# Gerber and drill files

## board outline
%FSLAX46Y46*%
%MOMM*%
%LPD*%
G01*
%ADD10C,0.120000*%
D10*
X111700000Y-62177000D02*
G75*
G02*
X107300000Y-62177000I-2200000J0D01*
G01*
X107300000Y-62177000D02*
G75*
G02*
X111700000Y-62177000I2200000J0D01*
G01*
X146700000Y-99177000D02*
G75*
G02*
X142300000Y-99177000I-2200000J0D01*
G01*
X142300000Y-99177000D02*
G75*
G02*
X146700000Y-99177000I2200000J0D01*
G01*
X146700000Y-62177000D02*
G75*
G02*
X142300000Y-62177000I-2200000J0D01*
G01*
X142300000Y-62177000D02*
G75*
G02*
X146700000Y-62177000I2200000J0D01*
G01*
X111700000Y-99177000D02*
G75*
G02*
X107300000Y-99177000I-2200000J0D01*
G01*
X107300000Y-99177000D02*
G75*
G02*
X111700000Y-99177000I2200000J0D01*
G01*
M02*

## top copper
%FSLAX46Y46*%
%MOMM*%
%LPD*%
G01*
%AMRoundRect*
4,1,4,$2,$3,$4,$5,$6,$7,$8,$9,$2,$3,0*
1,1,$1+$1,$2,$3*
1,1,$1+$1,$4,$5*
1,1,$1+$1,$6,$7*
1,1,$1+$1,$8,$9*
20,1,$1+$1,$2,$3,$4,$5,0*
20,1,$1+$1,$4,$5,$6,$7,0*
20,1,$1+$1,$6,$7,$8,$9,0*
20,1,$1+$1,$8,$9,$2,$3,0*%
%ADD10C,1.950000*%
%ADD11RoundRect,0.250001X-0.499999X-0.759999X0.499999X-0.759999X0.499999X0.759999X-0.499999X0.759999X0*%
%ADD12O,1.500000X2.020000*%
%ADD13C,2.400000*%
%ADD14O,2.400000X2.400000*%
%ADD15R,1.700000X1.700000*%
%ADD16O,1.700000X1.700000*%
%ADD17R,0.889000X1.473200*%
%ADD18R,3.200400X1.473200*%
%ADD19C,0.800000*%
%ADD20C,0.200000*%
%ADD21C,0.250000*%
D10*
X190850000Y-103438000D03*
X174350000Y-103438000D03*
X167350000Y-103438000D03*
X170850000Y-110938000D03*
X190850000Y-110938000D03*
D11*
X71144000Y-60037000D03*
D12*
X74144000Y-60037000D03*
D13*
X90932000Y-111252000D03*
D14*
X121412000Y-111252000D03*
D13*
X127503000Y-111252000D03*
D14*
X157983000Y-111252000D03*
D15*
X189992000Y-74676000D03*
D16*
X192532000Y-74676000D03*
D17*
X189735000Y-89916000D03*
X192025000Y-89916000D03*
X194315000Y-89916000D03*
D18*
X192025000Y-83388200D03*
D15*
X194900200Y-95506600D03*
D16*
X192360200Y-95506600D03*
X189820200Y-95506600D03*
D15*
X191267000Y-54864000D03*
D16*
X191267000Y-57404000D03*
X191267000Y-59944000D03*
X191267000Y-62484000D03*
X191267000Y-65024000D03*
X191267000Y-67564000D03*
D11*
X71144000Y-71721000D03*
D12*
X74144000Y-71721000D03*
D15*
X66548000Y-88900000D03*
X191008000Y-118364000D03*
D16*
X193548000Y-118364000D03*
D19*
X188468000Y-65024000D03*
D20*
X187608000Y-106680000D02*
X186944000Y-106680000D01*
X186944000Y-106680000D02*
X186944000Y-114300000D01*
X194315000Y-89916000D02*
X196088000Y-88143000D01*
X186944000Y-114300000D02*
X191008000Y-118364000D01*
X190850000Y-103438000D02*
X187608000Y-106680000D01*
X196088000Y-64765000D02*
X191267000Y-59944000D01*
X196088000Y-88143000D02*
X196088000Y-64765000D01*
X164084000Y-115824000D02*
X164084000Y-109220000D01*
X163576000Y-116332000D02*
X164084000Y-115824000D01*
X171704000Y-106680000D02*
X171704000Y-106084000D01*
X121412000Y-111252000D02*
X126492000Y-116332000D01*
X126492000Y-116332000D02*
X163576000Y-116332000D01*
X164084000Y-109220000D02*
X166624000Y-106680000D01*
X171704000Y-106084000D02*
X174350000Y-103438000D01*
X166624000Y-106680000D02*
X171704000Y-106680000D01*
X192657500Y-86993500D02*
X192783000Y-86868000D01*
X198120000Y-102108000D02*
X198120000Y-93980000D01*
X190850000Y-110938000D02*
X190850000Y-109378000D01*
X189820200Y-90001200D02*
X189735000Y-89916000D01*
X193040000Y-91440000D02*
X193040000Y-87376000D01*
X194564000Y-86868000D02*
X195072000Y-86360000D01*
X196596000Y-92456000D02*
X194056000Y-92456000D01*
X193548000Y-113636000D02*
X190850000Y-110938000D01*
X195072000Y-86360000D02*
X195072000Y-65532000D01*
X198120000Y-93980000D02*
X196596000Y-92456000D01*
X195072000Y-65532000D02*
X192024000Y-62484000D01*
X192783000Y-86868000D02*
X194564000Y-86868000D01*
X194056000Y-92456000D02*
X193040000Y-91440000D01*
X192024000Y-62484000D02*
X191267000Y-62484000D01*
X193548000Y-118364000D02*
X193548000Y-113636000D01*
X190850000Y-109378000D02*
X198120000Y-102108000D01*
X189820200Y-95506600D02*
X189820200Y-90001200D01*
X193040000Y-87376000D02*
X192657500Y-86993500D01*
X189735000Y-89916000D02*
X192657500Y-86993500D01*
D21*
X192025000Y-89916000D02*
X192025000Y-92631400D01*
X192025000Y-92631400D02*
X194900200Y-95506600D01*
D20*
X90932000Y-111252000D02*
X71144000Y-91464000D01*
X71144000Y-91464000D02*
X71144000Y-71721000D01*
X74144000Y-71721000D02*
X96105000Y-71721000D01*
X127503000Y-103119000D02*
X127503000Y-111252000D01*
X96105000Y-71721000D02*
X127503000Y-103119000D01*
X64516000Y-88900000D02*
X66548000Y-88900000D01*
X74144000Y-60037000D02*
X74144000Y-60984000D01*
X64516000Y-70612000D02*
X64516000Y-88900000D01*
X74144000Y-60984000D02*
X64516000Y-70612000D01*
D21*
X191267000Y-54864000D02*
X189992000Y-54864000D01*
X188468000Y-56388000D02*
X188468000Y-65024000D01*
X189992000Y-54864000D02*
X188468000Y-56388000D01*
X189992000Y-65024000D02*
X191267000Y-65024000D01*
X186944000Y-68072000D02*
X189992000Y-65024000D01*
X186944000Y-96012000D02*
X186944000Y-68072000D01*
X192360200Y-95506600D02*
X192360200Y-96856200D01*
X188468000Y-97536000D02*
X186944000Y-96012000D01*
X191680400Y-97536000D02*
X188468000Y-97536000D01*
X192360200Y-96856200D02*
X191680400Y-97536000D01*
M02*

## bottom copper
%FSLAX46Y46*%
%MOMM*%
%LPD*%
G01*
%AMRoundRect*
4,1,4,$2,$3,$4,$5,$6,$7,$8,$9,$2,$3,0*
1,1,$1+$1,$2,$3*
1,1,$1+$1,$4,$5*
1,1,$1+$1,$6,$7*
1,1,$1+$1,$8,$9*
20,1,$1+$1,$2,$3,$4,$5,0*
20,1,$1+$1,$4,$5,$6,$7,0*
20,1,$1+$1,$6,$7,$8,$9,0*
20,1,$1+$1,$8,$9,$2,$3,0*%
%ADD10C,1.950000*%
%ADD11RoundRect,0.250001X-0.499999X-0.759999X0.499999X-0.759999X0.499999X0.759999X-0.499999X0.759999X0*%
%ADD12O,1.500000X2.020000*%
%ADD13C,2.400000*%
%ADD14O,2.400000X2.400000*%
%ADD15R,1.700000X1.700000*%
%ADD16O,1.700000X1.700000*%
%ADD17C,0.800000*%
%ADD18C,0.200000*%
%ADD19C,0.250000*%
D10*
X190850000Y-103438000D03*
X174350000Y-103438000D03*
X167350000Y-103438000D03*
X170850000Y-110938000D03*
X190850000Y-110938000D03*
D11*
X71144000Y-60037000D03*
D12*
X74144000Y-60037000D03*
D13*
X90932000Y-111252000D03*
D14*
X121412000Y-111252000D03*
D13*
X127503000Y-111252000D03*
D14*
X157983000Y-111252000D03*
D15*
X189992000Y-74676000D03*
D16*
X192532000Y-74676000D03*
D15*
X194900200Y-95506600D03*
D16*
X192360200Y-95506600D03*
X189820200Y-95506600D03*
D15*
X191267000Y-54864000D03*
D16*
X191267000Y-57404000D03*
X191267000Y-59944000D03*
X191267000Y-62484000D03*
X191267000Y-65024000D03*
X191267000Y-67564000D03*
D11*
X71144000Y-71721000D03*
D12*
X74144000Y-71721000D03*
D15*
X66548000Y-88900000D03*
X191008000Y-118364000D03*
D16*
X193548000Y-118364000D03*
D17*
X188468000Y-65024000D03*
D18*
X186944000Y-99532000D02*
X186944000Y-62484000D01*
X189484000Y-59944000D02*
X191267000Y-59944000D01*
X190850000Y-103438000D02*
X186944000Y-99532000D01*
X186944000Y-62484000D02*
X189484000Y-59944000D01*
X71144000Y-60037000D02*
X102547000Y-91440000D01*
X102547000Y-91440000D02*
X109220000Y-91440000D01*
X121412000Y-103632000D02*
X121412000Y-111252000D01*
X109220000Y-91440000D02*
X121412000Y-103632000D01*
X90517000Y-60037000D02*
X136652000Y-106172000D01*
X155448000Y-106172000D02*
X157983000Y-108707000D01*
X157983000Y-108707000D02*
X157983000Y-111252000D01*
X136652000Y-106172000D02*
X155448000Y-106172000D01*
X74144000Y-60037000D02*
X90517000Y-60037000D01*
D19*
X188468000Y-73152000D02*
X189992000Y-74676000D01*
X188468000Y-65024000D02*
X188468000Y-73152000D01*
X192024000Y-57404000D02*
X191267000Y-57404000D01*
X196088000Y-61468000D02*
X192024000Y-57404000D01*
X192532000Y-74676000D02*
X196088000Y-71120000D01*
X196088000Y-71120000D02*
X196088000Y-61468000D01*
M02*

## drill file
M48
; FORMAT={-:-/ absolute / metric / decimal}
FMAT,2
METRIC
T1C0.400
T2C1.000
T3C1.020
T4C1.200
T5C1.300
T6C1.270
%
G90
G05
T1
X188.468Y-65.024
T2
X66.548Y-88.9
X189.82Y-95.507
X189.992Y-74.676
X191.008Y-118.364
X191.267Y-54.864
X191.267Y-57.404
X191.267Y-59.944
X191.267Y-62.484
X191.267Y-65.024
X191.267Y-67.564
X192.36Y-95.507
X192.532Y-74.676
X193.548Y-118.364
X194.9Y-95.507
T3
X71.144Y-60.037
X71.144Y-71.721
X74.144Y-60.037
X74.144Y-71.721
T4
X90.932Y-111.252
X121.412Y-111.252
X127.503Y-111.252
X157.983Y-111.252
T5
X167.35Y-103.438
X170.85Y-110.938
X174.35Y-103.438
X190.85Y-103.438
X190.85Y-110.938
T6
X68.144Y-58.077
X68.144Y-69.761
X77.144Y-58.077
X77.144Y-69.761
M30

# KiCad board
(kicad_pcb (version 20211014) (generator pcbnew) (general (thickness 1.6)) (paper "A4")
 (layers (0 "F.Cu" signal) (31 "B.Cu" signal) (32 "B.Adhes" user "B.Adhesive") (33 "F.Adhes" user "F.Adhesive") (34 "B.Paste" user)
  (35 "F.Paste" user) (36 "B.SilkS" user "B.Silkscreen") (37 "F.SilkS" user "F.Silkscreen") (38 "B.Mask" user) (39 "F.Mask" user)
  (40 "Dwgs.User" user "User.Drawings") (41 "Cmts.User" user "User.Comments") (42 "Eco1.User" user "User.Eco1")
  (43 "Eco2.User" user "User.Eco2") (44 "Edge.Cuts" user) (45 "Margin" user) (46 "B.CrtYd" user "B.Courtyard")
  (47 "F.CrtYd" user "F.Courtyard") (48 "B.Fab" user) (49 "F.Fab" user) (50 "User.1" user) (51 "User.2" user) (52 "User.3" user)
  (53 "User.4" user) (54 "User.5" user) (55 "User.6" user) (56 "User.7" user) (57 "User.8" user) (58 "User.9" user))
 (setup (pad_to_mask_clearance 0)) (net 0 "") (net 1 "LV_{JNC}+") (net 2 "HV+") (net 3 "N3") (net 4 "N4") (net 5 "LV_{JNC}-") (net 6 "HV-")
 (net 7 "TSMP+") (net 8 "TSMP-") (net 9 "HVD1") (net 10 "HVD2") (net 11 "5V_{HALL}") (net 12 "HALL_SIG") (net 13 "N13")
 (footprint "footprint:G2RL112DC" (layer "F.Cu") (at 190.85 103.438 180)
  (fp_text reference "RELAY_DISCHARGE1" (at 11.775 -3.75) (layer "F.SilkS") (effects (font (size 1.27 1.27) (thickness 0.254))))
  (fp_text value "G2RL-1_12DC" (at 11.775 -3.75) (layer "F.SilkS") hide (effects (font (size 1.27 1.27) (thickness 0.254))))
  (pad "1" thru_hole circle (at 0 0 180) (size 1.95 1.95) (drill 1.3) (layers *.Cu *.Mask) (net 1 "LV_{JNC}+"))
  (pad "2" thru_hole circle (at 16.5 0 180) (size 1.95 1.95) (drill 1.3) (layers *.Cu *.Mask) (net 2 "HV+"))
  (pad "3" thru_hole circle (at 23.5 0 180) (size 1.95 1.95) (drill 1.3) (layers *.Cu *.Mask) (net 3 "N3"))
  (pad "4" thru_hole circle (at 20 -7.5 180) (size 1.95 1.95) (drill 1.3) (layers *.Cu *.Mask) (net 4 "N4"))
  (pad "5" thru_hole circle (at 0 -7.5 180) (size 1.95 1.95) (drill 1.3) (layers *.Cu *.Mask) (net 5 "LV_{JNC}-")))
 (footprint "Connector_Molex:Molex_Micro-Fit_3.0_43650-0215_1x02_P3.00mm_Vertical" (layer "F.Cu") (at 71.144 60.037)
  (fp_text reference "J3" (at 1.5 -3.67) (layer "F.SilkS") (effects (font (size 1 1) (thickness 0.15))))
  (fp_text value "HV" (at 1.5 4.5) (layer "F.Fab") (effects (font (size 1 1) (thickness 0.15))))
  (pad "" np_thru_hole circle (at -3 -1.96) (size 1.27 1.27) (drill 1.27) (layers *.Cu *.Mask))
  (pad "" np_thru_hole circle (at 6 -1.96) (size 1.27 1.27) (drill 1.27) (layers *.Cu *.Mask))
  (pad "1" thru_hole roundrect (at 0 0) (size 1.5 2.02) (drill 1.02) (layers *.Cu *.Mask) (roundrect_rratio 0.166667) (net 2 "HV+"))
  (pad "2" thru_hole oval (at 3 0) (size 1.5 2.02) (drill 1.02) (layers *.Cu *.Mask) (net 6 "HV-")))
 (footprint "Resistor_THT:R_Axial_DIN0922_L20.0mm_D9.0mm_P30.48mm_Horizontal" (layer "F.Cu") (at 90.932 111.252)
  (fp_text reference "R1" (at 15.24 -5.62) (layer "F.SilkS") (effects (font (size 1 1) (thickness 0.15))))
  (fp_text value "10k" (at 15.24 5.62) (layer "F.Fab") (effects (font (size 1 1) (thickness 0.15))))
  (pad "1" thru_hole circle (at 0 0) (size 2.4 2.4) (drill 1.2) (layers *.Cu *.Mask) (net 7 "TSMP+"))
  (pad "2" thru_hole oval (at 30.48 0) (size 2.4 2.4) (drill 1.2) (layers *.Cu *.Mask) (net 2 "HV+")))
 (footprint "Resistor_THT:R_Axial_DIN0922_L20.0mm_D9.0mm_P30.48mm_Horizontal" (layer "F.Cu") (at 127.503 111.252)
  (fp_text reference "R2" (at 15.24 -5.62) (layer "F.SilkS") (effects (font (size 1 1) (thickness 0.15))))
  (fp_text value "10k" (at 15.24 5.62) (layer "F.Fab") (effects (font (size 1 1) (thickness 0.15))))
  (pad "1" thru_hole circle (at 0 0) (size 2.4 2.4) (drill 1.2) (layers *.Cu *.Mask) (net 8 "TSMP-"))
  (pad "2" thru_hole oval (at 30.48 0) (size 2.4 2.4) (drill 1.2) (layers *.Cu *.Mask) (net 6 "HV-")))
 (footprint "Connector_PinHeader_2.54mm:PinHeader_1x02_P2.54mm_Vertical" (layer "F.Cu") (at 189.992 74.676 90)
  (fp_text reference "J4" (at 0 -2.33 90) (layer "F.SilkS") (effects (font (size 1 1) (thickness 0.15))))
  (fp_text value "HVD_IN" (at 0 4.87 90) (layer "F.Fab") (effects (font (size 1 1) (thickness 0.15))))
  (pad "1" thru_hole rect (at 0 0 90) (size 1.7 1.7) (drill 1) (layers *.Cu *.Mask) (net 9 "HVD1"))
  (pad "2" thru_hole oval (at 0 2.54 90) (size 1.7 1.7) (drill 1) (layers *.Cu *.Mask) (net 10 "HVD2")))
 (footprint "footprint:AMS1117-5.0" (layer "F.Cu") (at 192.025 86.6521)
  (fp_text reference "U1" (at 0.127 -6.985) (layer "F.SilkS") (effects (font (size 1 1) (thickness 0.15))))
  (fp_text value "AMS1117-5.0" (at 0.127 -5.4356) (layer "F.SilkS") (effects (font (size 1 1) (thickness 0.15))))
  (pad "1" smd rect (at -2.29 3.2639) (size 0.889 1.4732) (layers "F.Cu" "F.Paste" "F.Mask") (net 5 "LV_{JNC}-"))
  (pad "2" smd rect (at 0 3.2639) (size 0.889 1.4732) (layers "F.Cu" "F.Paste" "F.Mask") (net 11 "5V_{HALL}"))
  (pad "3" smd rect (at 2.29 3.2639) (size 0.889 1.4732) (layers "F.Cu" "F.Paste" "F.Mask") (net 1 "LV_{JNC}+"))
  (pad "4" smd rect (at 0 -3.2639) (size 3.2004 1.4732) (layers "F.Cu" "F.Paste" "F.Mask")))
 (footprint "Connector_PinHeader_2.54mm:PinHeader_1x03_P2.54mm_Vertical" (layer "F.Cu") (at 194.9002 95.5066 -90)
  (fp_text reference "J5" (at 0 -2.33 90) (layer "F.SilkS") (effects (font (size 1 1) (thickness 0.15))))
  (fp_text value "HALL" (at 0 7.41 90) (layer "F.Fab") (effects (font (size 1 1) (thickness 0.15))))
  (pad "1" thru_hole rect (at 0 0 270) (size 1.7 1.7) (drill 1) (layers *.Cu *.Mask) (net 11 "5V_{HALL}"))
  (pad "2" thru_hole oval (at 0 2.54 270) (size 1.7 1.7) (drill 1) (layers *.Cu *.Mask) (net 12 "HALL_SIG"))
  (pad "3" thru_hole oval (at 0 5.08 270) (size 1.7 1.7) (drill 1) (layers *.Cu *.Mask) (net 5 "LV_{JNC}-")))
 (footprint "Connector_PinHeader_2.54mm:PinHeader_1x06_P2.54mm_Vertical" (layer "F.Cu") (at 191.267 54.864)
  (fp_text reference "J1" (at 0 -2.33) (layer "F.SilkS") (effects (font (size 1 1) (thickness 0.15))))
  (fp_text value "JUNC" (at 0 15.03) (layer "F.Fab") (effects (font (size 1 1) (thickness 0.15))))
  (pad "1" thru_hole rect (at 0 0) (size 1.7 1.7) (drill 1) (layers *.Cu *.Mask) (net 9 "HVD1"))
  (pad "2" thru_hole oval (at 0 2.54) (size 1.7 1.7) (drill 1) (layers *.Cu *.Mask) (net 10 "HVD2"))
  (pad "3" thru_hole oval (at 0 5.08) (size 1.7 1.7) (drill 1) (layers *.Cu *.Mask) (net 1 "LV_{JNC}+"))
  (pad "4" thru_hole oval (at 0 7.62) (size 1.7 1.7) (drill 1) (layers *.Cu *.Mask) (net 5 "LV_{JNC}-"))
  (pad "5" thru_hole oval (at 0 10.16) (size 1.7 1.7) (drill 1) (layers *.Cu *.Mask) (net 12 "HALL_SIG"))
  (pad "6" thru_hole oval (at 0 12.7) (size 1.7 1.7) (drill 1) (layers *.Cu *.Mask) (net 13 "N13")))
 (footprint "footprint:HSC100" (layer "F.Cu") (at 94.25 104.427)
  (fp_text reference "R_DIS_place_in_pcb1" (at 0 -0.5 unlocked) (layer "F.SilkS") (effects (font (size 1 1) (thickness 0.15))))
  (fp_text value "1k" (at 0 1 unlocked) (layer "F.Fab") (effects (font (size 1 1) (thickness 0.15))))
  (fp_circle (center 15.25 -42.25) (end 17.45 -42.25) (layer "Edge.Cuts") (width 0.12) (fill none))
  (fp_circle (center 50.25 -5.25) (end 52.45 -5.25) (layer "Edge.Cuts") (width 0.12) (fill none))
  (fp_circle (center 50.25 -42.25) (end 52.45 -42.25) (layer "Edge.Cuts") (width 0.12) (fill none))
  (fp_circle (center 15.25 -5.25) (end 17.45 -5.25) (layer "Edge.Cuts") (width 0.12) (fill none)))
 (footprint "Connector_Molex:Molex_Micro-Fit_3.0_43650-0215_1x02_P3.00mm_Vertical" (layer "F.Cu") (at 71.144 71.721)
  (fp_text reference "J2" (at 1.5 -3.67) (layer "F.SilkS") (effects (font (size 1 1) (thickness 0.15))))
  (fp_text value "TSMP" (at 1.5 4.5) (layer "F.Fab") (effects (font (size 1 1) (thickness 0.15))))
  (pad "" np_thru_hole circle (at -3 -1.96) (size 1.27 1.27) (drill 1.27) (layers *.Cu *.Mask))
  (pad "" np_thru_hole circle (at 6 -1.96) (size 1.27 1.27) (drill 1.27) (layers *.Cu *.Mask))
  (pad "1" thru_hole roundrect (at 0 0) (size 1.5 2.02) (drill 1.02) (layers *.Cu *.Mask) (roundrect_rratio 0.166667) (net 7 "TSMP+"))
  (pad "2" thru_hole oval (at 3 0) (size 1.5 2.02) (drill 1.02) (layers *.Cu *.Mask) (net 8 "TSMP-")))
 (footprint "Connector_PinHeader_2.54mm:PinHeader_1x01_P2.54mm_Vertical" (layer "F.Cu") (at 66.548 88.9)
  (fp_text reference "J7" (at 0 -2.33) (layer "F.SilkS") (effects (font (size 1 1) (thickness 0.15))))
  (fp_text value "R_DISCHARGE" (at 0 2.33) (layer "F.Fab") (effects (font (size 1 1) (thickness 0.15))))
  (pad "1" thru_hole rect (at 0 0) (size 1.7 1.7) (drill 1) (layers *.Cu *.Mask) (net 6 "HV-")))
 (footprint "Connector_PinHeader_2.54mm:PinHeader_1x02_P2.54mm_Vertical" (layer "F.Cu") (at 191.008 118.364 90)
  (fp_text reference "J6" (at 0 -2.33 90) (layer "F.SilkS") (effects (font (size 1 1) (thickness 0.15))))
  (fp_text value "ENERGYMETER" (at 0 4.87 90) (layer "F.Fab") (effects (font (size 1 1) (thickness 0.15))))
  (pad "1" thru_hole rect (at 0 0 90) (size 1.7 1.7) (drill 1) (layers *.Cu *.Mask) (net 1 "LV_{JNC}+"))
  (pad "2" thru_hole oval (at 0 2.54 90) (size 1.7 1.7) (drill 1) (layers *.Cu *.Mask) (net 5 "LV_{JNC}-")))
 (segment (start 187.608 106.68) (end 186.944 106.68) (width 0.2) (layer "F.Cu") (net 1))
 (segment (start 186.944 106.68) (end 186.944 114.3) (width 0.2) (layer "F.Cu") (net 1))
 (segment (start 194.315 89.916) (end 196.088 88.143) (width 0.2) (layer "F.Cu") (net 1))
 (segment (start 186.944 114.3) (end 191.008 118.364) (width 0.2) (layer "F.Cu") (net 1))
 (segment (start 190.85 103.438) (end 187.608 106.68) (width 0.2) (layer "F.Cu") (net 1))
 (segment (start 196.088 64.765) (end 191.267 59.944) (width 0.2) (layer "F.Cu") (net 1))
 (segment (start 196.088 88.143) (end 196.088 64.765) (width 0.2) (layer "F.Cu") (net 1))
 (segment (start 186.944 99.532) (end 186.944 62.484) (width 0.2) (layer "B.Cu") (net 1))
 (segment (start 189.484 59.944) (end 191.267 59.944) (width 0.2) (layer "B.Cu") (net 1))
 (segment (start 190.85 103.438) (end 186.944 99.532) (width 0.2) (layer "B.Cu") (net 1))
 (segment (start 186.944 62.484) (end 189.484 59.944) (width 0.2) (layer "B.Cu") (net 1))
 (segment (start 164.084 115.824) (end 164.084 109.22) (width 0.2) (layer "F.Cu") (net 2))
 (segment (start 163.576 116.332) (end 164.084 115.824) (width 0.2) (layer "F.Cu") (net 2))
 (segment (start 171.704 106.68) (end 171.704 106.084) (width 0.2) (layer "F.Cu") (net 2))
 (segment (start 121.412 111.252) (end 126.492 116.332) (width 0.2) (layer "F.Cu") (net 2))
 (segment (start 126.492 116.332) (end 163.576 116.332) (width 0.2) (layer "F.Cu") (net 2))
 (segment (start 164.084 109.22) (end 166.624 106.68) (width 0.2) (layer "F.Cu") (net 2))
 (segment (start 171.704 106.084) (end 174.35 103.438) (width 0.2) (layer "F.Cu") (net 2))
 (segment (start 166.624 106.68) (end 171.704 106.68) (width 0.2) (layer "F.Cu") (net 2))
 (segment (start 71.144 60.037) (end 102.547 91.44) (width 0.2) (layer "B.Cu") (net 2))
 (segment (start 102.547 91.44) (end 109.22 91.44) (width 0.2) (layer "B.Cu") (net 2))
 (segment (start 121.412 103.632) (end 121.412 111.252) (width 0.2) (layer "B.Cu") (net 2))
 (segment (start 109.22 91.44) (end 121.412 103.632) (width 0.2) (layer "B.Cu") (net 2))
 (segment (start 192.6575 86.9935) (end 192.783 86.868) (width 0.2) (layer "F.Cu") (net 5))
 (segment (start 198.12 102.108) (end 198.12 93.98) (width 0.2) (layer "F.Cu") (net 5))
 (segment (start 190.85 110.938) (end 190.85 109.378) (width 0.2) (layer "F.Cu") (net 5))
 (segment (start 189.8202 90.0012) (end 189.735 89.916) (width 0.2) (layer "F.Cu") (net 5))
 (segment (start 193.04 91.44) (end 193.04 87.376) (width 0.2) (layer "F.Cu") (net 5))
 (segment (start 194.564 86.868) (end 195.072 86.36) (width 0.2) (layer "F.Cu") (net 5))
 (segment (start 196.596 92.456) (end 194.056 92.456) (width 0.2) (layer "F.Cu") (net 5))
 (segment (start 193.548 113.636) (end 190.85 110.938) (width 0.2) (layer "F.Cu") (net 5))
 (segment (start 195.072 86.36) (end 195.072 65.532) (width 0.2) (layer "F.Cu") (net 5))
 (segment (start 198.12 93.98) (end 196.596 92.456) (width 0.2) (layer "F.Cu") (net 5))
 (segment (start 195.072 65.532) (end 192.024 62.484) (width 0.2) (layer "F.Cu") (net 5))
 (segment (start 192.783 86.868) (end 194.564 86.868) (width 0.2) (layer "F.Cu") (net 5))
 (segment (start 194.056 92.456) (end 193.04 91.44) (width 0.2) (layer "F.Cu") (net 5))
 (segment (start 192.024 62.484) (end 191.267 62.484) (width 0.2) (layer "F.Cu") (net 5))
 (segment (start 193.548 118.364) (end 193.548 113.636) (width 0.2) (layer "F.Cu") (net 5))
 (segment (start 190.85 109.378) (end 198.12 102.108) (width 0.2) (layer "F.Cu") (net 5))
 (segment (start 189.8202 95.5066) (end 189.8202 90.0012) (width 0.2) (layer "F.Cu") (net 5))
 (segment (start 193.04 87.376) (end 192.6575 86.9935) (width 0.2) (layer "F.Cu") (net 5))
 (segment (start 189.735 89.916) (end 192.6575 86.9935) (width 0.2) (layer "F.Cu") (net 5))
 (segment (start 192.025 89.916) (end 192.025 92.6314) (width 0.25) (layer "F.Cu") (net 11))
 (segment (start 192.025 92.6314) (end 194.9002 95.5066) (width 0.25) (layer "F.Cu") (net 11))
 (segment (start 90.932 111.252) (end 71.144 91.464) (width 0.2) (layer "F.Cu") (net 7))
 (segment (start 71.144 91.464) (end 71.144 71.721) (width 0.2) (layer "F.Cu") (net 7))
 (segment (start 74.144 71.721) (end 96.105 71.721) (width 0.2) (layer "F.Cu") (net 8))
 (segment (start 127.503 103.119) (end 127.503 111.252) (width 0.2) (layer "F.Cu") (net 8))
 (segment (start 96.105 71.721) (end 127.503 103.119) (width 0.2) (layer "F.Cu") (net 8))
 (segment (start 64.516 88.9) (end 66.548 88.9) (width 0.2) (layer "F.Cu") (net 6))
 (segment (start 74.144 60.037) (end 74.144 60.984) (width 0.2) (layer "F.Cu") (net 6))
 (segment (start 64.516 70.612) (end 64.516 88.9) (width 0.2) (layer "F.Cu") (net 6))
 (segment (start 74.144 60.984) (end 64.516 70.612) (width 0.2) (layer "F.Cu") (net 6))
 (segment (start 90.517 60.037) (end 136.652 106.172) (width 0.2) (layer "B.Cu") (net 6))
 (segment (start 155.448 106.172) (end 157.983 108.707) (width 0.2) (layer "B.Cu") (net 6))
 (segment (start 157.983 108.707) (end 157.983 111.252) (width 0.2) (layer "B.Cu") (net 6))
 (segment (start 136.652 106.172) (end 155.448 106.172) (width 0.2) (layer "B.Cu") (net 6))
 (segment (start 74.144 60.037) (end 90.517 60.037) (width 0.2) (layer "B.Cu") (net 6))
 (segment (start 191.267 54.864) (end 189.992 54.864) (width 0.25) (layer "F.Cu") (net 9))
 (segment (start 188.468 56.388) (end 188.468 65.024) (width 0.25) (layer "F.Cu") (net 9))
 (segment (start 189.992 54.864) (end 188.468 56.388) (width 0.25) (layer "F.Cu") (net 9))
 (via (at 188.468 65.024) (size 0.8) (drill 0.4) (layers "F.Cu" "B.Cu") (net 9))
 (segment (start 188.468 73.152) (end 189.992 74.676) (width 0.25) (layer "B.Cu") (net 9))
 (segment (start 188.468 65.024) (end 188.468 73.152) (width 0.25) (layer "B.Cu") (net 9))
 (segment (start 192.024 57.404) (end 191.267 57.404) (width 0.25) (layer "B.Cu") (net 10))
 (segment (start 196.088 61.468) (end 192.024 57.404) (width 0.25) (layer "B.Cu") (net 10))
 (segment (start 192.532 74.676) (end 196.088 71.12) (width 0.25) (layer "B.Cu") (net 10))
 (segment (start 196.088 71.12) (end 196.088 61.468) (width 0.25) (layer "B.Cu") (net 10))
 (segment (start 189.992 65.024) (end 191.267 65.024) (width 0.25) (layer "F.Cu") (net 12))
 (segment (start 186.944 68.072) (end 189.992 65.024) (width 0.25) (layer "F.Cu") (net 12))
 (segment (start 186.944 96.012) (end 186.944 68.072) (width 0.25) (layer "F.Cu") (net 12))
 (segment (start 192.3602 95.5066) (end 192.3602 96.8562) (width 0.25) (layer "F.Cu") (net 12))
 (segment (start 188.468 97.536) (end 186.944 96.012) (width 0.25) (layer "F.Cu") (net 12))
 (segment (start 191.6804 97.536) (end 188.468 97.536) (width 0.25) (layer "F.Cu") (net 12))
 (segment (start 192.3602 96.8562) (end 191.6804 97.536) (width 0.25) (layer "F.Cu") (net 12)))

